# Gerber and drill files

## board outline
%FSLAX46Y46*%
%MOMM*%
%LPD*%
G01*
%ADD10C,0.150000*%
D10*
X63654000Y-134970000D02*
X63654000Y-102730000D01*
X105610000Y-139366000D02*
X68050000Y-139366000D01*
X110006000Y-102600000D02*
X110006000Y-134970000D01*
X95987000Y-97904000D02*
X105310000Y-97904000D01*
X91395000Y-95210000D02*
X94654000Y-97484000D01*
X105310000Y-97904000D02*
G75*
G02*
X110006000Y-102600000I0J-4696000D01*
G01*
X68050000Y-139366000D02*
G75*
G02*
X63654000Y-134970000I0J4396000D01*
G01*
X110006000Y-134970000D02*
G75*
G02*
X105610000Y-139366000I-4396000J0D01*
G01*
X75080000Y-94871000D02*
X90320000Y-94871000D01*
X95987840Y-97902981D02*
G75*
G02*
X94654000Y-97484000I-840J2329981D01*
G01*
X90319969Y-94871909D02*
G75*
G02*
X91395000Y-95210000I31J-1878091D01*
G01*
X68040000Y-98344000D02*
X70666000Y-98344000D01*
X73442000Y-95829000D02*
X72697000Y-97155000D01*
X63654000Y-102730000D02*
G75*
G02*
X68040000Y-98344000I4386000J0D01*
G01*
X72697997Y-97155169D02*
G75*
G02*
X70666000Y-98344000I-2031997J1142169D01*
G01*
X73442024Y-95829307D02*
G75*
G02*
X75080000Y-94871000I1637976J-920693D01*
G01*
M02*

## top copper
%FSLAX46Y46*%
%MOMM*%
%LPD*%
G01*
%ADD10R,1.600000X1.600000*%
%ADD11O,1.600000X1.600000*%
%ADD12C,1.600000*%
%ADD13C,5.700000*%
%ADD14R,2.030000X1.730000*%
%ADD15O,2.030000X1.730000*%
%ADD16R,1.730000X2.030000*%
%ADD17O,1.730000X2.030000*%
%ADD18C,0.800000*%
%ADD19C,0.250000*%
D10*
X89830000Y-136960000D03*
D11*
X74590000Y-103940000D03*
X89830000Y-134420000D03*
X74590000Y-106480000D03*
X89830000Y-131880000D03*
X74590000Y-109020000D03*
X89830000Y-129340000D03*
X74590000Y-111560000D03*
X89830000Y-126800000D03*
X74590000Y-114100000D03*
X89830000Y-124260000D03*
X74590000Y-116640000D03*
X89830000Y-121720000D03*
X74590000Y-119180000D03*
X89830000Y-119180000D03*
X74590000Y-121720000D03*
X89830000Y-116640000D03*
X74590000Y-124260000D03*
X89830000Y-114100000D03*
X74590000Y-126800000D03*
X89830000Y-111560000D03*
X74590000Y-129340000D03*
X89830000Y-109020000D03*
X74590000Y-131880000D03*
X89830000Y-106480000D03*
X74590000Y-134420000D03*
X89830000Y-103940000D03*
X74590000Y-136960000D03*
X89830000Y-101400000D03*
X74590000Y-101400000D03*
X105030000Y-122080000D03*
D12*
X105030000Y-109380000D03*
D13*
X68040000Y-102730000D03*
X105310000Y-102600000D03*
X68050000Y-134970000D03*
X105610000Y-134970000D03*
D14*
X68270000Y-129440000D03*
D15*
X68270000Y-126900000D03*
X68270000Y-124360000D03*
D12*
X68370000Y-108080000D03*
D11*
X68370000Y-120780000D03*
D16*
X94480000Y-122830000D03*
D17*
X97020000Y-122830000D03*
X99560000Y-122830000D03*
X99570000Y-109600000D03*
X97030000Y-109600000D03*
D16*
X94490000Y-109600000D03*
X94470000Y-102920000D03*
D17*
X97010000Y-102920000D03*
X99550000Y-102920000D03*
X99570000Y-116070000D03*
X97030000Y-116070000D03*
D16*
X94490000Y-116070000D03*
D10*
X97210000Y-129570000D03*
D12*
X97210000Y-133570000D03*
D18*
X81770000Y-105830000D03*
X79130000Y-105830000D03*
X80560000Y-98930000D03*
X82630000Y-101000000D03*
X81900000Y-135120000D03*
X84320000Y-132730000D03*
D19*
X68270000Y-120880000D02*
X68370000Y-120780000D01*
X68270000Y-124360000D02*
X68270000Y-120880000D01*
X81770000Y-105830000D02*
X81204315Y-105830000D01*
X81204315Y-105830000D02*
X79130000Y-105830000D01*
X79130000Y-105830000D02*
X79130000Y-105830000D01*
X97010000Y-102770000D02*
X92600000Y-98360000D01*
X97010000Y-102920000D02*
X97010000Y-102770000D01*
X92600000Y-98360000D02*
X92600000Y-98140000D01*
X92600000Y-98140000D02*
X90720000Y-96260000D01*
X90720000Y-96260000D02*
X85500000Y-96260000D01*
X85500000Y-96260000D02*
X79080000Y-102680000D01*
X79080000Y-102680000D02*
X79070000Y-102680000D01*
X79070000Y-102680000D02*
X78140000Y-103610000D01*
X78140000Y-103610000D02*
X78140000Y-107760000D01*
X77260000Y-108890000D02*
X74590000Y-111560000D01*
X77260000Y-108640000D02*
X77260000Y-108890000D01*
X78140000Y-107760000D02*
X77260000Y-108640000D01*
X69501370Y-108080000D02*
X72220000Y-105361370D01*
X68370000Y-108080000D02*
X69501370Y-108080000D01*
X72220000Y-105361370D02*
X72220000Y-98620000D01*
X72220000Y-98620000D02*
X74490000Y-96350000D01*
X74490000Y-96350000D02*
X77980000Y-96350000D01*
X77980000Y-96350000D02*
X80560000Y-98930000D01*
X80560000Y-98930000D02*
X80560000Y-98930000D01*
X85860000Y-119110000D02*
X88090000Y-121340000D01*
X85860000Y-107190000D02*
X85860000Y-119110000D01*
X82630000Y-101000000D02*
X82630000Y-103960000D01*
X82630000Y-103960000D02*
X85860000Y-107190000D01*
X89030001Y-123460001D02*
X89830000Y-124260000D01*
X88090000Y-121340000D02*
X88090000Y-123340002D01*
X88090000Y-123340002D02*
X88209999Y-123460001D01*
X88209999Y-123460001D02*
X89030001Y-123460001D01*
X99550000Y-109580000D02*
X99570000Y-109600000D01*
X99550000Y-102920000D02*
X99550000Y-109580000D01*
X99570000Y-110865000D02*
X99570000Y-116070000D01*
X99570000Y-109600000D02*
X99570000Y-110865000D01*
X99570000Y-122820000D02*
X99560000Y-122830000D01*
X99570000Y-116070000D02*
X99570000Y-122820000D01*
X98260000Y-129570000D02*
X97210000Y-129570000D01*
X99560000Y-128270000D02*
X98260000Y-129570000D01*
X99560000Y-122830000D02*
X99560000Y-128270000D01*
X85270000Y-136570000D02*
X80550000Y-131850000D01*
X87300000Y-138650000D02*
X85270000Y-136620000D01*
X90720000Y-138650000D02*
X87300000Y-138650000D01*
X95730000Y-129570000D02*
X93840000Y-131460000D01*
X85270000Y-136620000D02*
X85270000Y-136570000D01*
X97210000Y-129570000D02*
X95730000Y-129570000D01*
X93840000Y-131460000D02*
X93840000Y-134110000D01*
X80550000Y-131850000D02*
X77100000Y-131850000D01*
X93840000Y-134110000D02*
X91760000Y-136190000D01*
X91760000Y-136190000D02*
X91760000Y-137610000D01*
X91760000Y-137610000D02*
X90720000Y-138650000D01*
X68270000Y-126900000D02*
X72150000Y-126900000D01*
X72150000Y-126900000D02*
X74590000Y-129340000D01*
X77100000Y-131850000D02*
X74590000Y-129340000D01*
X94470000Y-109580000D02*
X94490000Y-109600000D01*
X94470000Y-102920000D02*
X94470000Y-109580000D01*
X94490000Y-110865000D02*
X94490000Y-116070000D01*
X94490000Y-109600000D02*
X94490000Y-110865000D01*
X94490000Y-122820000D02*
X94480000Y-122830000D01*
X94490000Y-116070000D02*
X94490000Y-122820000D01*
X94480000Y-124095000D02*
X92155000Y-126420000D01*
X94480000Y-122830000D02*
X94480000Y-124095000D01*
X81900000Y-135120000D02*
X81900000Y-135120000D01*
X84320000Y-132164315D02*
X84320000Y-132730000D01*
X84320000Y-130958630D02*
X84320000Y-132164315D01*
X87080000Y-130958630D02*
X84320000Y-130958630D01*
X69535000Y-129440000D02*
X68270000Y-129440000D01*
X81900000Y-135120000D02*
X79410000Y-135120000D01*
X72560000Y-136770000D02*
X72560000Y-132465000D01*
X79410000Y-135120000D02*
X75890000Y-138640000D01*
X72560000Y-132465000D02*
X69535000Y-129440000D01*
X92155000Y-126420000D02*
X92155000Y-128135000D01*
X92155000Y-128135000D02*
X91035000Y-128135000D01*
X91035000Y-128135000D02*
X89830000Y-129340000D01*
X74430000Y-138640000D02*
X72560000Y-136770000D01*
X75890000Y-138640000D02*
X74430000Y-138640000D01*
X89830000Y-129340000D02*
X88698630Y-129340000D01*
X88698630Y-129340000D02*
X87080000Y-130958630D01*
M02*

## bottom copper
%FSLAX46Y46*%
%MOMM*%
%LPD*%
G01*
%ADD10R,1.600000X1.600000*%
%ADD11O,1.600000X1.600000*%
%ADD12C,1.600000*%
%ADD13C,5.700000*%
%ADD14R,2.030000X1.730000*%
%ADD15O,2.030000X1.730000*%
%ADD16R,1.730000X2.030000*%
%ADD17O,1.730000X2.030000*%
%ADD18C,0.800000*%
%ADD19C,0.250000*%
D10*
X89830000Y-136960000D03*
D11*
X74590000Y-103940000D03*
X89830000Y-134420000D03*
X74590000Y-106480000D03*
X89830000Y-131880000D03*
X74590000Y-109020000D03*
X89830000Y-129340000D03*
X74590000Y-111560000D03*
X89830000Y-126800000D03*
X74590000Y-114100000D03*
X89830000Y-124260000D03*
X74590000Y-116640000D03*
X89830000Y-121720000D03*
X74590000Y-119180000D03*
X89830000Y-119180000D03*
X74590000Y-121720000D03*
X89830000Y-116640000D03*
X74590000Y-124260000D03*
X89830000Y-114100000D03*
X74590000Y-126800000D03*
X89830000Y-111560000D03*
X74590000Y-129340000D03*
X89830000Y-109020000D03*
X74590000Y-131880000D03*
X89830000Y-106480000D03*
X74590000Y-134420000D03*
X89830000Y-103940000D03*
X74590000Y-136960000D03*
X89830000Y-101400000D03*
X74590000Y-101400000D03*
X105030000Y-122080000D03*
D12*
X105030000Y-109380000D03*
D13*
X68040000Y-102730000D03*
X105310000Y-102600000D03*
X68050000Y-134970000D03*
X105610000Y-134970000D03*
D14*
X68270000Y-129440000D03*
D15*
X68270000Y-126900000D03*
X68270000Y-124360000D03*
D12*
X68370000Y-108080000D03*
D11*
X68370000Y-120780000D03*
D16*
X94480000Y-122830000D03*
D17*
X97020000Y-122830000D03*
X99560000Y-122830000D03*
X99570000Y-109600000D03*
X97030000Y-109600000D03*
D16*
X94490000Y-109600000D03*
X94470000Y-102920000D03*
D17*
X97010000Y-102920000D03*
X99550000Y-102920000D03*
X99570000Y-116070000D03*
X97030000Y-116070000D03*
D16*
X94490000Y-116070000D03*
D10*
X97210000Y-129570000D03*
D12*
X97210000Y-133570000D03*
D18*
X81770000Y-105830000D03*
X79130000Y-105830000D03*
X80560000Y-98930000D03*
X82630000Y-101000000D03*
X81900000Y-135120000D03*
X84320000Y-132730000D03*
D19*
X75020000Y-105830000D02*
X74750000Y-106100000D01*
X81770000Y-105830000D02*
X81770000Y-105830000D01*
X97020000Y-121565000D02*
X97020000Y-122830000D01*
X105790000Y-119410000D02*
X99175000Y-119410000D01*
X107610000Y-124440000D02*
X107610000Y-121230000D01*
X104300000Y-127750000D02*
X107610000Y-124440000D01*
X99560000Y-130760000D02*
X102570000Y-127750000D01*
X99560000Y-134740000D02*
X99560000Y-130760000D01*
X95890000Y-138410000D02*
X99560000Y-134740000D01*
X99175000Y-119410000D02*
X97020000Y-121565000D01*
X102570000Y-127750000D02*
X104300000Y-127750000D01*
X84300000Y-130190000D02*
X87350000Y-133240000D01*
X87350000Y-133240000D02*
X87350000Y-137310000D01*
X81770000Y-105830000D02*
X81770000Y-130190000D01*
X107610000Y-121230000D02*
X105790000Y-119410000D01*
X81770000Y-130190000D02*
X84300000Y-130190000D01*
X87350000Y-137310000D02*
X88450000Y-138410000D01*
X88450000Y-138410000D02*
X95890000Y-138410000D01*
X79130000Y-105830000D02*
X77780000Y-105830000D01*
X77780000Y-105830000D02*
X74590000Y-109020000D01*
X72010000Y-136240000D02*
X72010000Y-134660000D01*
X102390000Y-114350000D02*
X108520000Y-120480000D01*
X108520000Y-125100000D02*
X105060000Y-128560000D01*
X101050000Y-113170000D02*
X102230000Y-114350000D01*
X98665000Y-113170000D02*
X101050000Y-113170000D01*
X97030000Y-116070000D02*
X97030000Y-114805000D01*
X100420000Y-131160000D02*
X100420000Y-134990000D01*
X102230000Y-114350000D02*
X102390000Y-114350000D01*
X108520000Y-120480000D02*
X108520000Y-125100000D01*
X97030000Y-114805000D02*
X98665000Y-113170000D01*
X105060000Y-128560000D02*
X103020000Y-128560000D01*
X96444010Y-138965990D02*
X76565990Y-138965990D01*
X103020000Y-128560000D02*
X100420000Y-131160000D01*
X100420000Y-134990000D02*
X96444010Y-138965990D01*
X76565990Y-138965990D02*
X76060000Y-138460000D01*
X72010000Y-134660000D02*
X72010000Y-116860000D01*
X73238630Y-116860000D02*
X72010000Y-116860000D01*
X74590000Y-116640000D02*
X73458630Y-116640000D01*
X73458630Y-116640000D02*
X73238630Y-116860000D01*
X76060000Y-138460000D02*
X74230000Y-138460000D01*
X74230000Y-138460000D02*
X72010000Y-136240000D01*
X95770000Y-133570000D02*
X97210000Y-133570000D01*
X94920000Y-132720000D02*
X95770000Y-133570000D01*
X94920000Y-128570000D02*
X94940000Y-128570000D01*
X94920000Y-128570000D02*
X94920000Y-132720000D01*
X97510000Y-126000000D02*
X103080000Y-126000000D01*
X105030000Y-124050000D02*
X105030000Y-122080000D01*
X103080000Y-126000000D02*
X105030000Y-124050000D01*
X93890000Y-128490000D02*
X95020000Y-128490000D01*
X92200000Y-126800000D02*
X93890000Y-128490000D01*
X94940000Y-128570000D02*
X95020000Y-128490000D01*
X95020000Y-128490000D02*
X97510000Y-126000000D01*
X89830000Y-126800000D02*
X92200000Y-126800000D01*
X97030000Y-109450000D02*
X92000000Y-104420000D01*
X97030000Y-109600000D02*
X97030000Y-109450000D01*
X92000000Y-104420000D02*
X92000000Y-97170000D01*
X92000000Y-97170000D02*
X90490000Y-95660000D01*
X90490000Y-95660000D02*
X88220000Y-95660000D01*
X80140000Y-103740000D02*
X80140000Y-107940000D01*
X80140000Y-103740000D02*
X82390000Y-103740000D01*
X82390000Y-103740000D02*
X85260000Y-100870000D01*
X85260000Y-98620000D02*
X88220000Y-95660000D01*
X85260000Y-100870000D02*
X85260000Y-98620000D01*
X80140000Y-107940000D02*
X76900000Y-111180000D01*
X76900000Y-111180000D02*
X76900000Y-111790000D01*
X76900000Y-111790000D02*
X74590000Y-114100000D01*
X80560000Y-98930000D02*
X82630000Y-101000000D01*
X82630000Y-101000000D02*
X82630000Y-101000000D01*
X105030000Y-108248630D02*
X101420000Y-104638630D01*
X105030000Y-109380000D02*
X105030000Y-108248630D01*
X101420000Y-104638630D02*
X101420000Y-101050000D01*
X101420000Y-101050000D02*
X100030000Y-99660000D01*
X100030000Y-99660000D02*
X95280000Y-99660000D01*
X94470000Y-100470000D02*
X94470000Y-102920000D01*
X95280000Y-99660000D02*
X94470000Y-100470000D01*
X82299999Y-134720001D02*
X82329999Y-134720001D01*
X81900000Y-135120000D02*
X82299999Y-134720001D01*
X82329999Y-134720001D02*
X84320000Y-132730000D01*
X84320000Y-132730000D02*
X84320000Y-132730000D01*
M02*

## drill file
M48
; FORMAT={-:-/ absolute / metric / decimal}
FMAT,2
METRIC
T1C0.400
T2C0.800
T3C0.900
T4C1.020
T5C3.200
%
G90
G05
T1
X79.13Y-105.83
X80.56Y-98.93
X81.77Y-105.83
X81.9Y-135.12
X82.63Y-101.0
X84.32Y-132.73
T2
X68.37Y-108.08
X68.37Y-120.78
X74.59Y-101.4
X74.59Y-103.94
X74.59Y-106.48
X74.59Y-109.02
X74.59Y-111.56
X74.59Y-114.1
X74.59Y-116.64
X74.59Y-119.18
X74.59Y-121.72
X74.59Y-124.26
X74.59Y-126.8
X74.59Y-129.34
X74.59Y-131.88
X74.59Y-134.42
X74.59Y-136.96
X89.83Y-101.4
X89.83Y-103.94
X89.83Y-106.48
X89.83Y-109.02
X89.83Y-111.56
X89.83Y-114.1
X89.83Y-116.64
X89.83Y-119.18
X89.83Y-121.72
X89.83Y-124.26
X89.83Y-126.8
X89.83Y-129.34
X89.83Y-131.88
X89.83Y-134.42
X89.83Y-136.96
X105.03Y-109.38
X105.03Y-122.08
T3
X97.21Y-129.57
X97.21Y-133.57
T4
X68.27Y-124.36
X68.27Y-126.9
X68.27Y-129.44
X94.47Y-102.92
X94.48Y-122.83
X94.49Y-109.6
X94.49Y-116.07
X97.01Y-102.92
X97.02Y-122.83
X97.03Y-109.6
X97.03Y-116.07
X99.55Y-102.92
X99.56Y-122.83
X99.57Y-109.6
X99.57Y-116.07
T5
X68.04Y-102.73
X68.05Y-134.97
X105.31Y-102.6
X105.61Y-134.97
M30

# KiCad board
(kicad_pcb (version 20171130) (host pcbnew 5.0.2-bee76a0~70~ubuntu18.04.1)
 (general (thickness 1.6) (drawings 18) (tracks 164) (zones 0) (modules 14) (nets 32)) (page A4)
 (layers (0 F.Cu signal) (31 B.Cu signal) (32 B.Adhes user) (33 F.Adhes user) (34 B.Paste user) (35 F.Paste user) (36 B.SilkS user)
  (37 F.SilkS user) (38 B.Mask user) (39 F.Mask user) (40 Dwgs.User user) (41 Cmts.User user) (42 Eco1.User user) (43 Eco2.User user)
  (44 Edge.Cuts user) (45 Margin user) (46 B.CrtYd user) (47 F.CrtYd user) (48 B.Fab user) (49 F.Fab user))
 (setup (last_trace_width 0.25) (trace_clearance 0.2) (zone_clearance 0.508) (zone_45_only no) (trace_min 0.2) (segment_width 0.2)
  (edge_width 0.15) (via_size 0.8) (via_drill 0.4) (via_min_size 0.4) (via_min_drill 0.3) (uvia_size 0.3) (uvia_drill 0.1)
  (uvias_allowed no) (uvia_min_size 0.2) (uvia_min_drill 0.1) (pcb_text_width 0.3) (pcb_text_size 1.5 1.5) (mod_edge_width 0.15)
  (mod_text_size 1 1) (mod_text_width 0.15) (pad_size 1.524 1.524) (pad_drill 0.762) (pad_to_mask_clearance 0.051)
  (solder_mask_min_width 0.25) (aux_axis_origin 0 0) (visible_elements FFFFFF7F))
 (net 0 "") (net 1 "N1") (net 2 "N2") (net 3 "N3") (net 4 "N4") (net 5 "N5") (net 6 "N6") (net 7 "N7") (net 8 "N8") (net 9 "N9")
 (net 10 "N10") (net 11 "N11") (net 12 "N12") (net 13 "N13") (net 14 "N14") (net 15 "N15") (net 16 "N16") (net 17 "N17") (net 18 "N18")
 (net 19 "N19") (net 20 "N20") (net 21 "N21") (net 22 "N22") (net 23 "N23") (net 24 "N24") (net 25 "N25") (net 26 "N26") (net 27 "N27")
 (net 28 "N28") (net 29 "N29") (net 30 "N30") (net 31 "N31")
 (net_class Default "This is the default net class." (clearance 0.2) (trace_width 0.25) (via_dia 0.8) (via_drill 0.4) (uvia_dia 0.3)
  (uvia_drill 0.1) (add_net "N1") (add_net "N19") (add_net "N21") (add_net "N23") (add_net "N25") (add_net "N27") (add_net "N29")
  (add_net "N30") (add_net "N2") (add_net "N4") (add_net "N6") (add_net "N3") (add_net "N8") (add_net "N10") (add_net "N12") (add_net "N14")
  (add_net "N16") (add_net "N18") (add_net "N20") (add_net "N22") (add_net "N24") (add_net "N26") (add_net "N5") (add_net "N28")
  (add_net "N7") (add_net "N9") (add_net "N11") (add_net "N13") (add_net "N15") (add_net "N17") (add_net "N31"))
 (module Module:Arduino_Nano (layer F.Cu) (at 89.83 136.96 180)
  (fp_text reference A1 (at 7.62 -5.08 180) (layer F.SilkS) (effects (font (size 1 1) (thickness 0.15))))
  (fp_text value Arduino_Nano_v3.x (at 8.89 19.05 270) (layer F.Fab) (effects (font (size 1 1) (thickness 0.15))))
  (pad 1 thru_hole rect (at 0 0 180) (size 1.6 1.6) (drill 0.8) (layers *.Cu *.Mask) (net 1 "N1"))
  (pad 17 thru_hole oval (at 15.24 33.02 180) (size 1.6 1.6) (drill 0.8) (layers *.Cu *.Mask) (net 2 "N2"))
  (pad 2 thru_hole oval (at 0 2.54 180) (size 1.6 1.6) (drill 0.8) (layers *.Cu *.Mask) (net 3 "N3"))
  (pad 18 thru_hole oval (at 15.24 30.48 180) (size 1.6 1.6) (drill 0.8) (layers *.Cu *.Mask) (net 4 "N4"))
  (pad 3 thru_hole oval (at 0 5.08 180) (size 1.6 1.6) (drill 0.8) (layers *.Cu *.Mask) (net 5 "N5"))
  (pad 19 thru_hole oval (at 15.24 27.94 180) (size 1.6 1.6) (drill 0.8) (layers *.Cu *.Mask) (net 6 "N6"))
  (pad 4 thru_hole oval (at 0 7.62 180) (size 1.6 1.6) (drill 0.8) (layers *.Cu *.Mask) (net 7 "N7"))
  (pad 20 thru_hole oval (at 15.24 25.4 180) (size 1.6 1.6) (drill 0.8) (layers *.Cu *.Mask) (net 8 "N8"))
  (pad 5 thru_hole oval (at 0 10.16 180) (size 1.6 1.6) (drill 0.8) (layers *.Cu *.Mask) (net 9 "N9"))
  (pad 21 thru_hole oval (at 15.24 22.86 180) (size 1.6 1.6) (drill 0.8) (layers *.Cu *.Mask) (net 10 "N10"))
  (pad 6 thru_hole oval (at 0 12.7 180) (size 1.6 1.6) (drill 0.8) (layers *.Cu *.Mask) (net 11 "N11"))
  (pad 22 thru_hole oval (at 15.24 20.32 180) (size 1.6 1.6) (drill 0.8) (layers *.Cu *.Mask) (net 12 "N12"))
  (pad 7 thru_hole oval (at 0 15.24 180) (size 1.6 1.6) (drill 0.8) (layers *.Cu *.Mask) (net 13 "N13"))
  (pad 23 thru_hole oval (at 15.24 17.78 180) (size 1.6 1.6) (drill 0.8) (layers *.Cu *.Mask) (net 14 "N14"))
  (pad 8 thru_hole oval (at 0 17.78 180) (size 1.6 1.6) (drill 0.8) (layers *.Cu *.Mask) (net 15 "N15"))
  (pad 24 thru_hole oval (at 15.24 15.24 180) (size 1.6 1.6) (drill 0.8) (layers *.Cu *.Mask) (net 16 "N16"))
  (pad 9 thru_hole oval (at 0 20.32 180) (size 1.6 1.6) (drill 0.8) (layers *.Cu *.Mask) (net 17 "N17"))
  (pad 25 thru_hole oval (at 15.24 12.7 180) (size 1.6 1.6) (drill 0.8) (layers *.Cu *.Mask) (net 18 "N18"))
  (pad 10 thru_hole oval (at 0 22.86 180) (size 1.6 1.6) (drill 0.8) (layers *.Cu *.Mask) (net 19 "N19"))
  (pad 26 thru_hole oval (at 15.24 10.16 180) (size 1.6 1.6) (drill 0.8) (layers *.Cu *.Mask) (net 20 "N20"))
  (pad 11 thru_hole oval (at 0 25.4 180) (size 1.6 1.6) (drill 0.8) (layers *.Cu *.Mask) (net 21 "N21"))
  (pad 27 thru_hole oval (at 15.24 7.62 180) (size 1.6 1.6) (drill 0.8) (layers *.Cu *.Mask) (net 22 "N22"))
  (pad 12 thru_hole oval (at 0 27.94 180) (size 1.6 1.6) (drill 0.8) (layers *.Cu *.Mask) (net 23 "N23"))
  (pad 28 thru_hole oval (at 15.24 5.08 180) (size 1.6 1.6) (drill 0.8) (layers *.Cu *.Mask) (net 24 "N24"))
  (pad 13 thru_hole oval (at 0 30.48 180) (size 1.6 1.6) (drill 0.8) (layers *.Cu *.Mask) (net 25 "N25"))
  (pad 29 thru_hole oval (at 15.24 2.54 180) (size 1.6 1.6) (drill 0.8) (layers *.Cu *.Mask) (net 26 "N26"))
  (pad 14 thru_hole oval (at 0 33.02 180) (size 1.6 1.6) (drill 0.8) (layers *.Cu *.Mask) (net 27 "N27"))
  (pad 30 thru_hole oval (at 15.24 0 180) (size 1.6 1.6) (drill 0.8) (layers *.Cu *.Mask) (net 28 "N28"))
  (pad 15 thru_hole oval (at 0 35.56 180) (size 1.6 1.6) (drill 0.8) (layers *.Cu *.Mask) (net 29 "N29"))
  (pad 16 thru_hole oval (at 15.24 35.56 180) (size 1.6 1.6) (drill 0.8) (layers *.Cu *.Mask) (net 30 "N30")))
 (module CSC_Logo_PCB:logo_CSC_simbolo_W (layer F.Cu) (at 81.88 125.63)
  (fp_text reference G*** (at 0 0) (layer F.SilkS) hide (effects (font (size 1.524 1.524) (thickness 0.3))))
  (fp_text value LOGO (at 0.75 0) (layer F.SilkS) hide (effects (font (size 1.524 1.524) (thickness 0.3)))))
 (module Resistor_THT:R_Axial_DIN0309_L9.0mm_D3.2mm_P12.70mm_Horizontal (layer F.Cu) (at 105.03 109.38 270)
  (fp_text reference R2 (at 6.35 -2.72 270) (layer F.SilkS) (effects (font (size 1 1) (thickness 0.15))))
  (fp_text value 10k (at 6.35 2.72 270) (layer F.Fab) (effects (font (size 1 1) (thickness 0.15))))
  (pad 2 thru_hole oval (at 12.7 0 270) (size 1.6 1.6) (drill 0.8) (layers *.Cu *.Mask) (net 9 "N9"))
  (pad 1 thru_hole circle (at 0 0 270) (size 1.6 1.6) (drill 0.8) (layers *.Cu *.Mask) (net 7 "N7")))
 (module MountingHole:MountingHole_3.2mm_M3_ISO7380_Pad (layer F.Cu) (at 68.04 102.73)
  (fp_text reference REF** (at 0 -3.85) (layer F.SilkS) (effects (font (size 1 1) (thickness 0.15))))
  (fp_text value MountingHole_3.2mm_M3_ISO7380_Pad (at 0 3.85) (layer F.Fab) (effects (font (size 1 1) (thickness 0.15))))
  (pad 1 thru_hole circle (at 0 0) (size 5.7 5.7) (drill 3.2) (layers *.Cu *.Mask)))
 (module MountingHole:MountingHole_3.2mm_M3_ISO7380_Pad (layer F.Cu) (at 105.31 102.6)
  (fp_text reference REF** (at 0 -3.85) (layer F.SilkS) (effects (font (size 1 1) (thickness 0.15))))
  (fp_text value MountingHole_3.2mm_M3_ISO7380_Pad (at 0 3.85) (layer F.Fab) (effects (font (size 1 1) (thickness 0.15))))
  (pad 1 thru_hole circle (at 0 0) (size 5.7 5.7) (drill 3.2) (layers *.Cu *.Mask)))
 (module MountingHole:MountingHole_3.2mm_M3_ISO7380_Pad (layer F.Cu) (at 68.05 134.97)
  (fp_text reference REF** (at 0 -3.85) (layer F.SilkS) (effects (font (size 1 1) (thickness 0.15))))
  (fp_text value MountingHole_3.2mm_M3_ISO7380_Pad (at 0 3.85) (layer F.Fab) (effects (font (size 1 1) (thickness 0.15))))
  (pad 1 thru_hole circle (at 0 0) (size 5.7 5.7) (drill 3.2) (layers *.Cu *.Mask)))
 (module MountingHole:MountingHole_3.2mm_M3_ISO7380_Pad (layer F.Cu) (at 105.61 134.97)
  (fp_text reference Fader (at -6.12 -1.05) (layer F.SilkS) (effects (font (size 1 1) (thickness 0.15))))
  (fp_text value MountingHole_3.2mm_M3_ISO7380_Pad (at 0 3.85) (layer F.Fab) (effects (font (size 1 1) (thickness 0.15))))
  (pad 1 thru_hole circle (at 0 0) (size 5.7 5.7) (drill 3.2) (layers *.Cu *.Mask)))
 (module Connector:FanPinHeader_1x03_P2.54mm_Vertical (layer F.Cu) (at 68.27 129.44 90)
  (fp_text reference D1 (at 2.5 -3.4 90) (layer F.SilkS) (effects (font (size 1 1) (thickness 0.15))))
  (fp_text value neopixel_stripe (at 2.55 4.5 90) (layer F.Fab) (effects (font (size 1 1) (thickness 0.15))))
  (pad 1 thru_hole rect (at 0 0 180) (size 2.03 1.73) (drill 1.02) (layers *.Cu *.Mask) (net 7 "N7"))
  (pad 2 thru_hole oval (at 2.54 0 180) (size 2.03 1.73) (drill 1.02) (layers *.Cu *.Mask) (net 22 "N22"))
  (pad 3 thru_hole oval (at 5.08 0 180) (size 2.03 1.73) (drill 1.02) (layers *.Cu *.Mask) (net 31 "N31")))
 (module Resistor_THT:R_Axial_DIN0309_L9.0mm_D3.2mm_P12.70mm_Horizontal (layer F.Cu) (at 68.37 108.08 270)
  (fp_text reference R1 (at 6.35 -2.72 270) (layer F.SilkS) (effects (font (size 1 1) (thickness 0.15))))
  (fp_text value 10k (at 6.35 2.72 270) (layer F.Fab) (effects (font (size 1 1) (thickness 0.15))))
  (pad 1 thru_hole circle (at 0 0 270) (size 1.6 1.6) (drill 0.8) (layers *.Cu *.Mask) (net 11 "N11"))
  (pad 2 thru_hole oval (at 12.7 0 270) (size 1.6 1.6) (drill 0.8) (layers *.Cu *.Mask) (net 31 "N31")))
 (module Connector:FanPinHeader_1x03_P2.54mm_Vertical (layer F.Cu) (at 94.48 122.83)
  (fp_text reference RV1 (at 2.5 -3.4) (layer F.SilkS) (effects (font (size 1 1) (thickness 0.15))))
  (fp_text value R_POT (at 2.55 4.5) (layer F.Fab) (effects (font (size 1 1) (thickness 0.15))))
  (pad 1 thru_hole rect (at 0 0 90) (size 2.03 1.73) (drill 1.02) (layers *.Cu *.Mask) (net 7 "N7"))
  (pad 2 thru_hole oval (at 2.54 0 90) (size 2.03 1.73) (drill 1.02) (layers *.Cu *.Mask) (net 6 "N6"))
  (pad 3 thru_hole oval (at 5.08 0 90) (size 2.03 1.73) (drill 1.02) (layers *.Cu *.Mask) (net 22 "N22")))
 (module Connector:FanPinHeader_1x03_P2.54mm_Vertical (layer F.Cu) (at 94.49 109.6)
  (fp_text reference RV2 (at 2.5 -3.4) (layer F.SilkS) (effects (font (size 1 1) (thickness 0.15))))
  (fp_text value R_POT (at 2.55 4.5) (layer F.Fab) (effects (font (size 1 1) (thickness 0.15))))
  (pad 3 thru_hole oval (at 5.08 0 90) (size 2.03 1.73) (drill 1.02) (layers *.Cu *.Mask) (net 22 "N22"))
  (pad 2 thru_hole oval (at 2.54 0 90) (size 2.03 1.73) (drill 1.02) (layers *.Cu *.Mask) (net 10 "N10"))
  (pad 1 thru_hole rect (at 0 0 90) (size 2.03 1.73) (drill 1.02) (layers *.Cu *.Mask) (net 7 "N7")))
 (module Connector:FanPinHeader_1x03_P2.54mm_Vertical (layer F.Cu) (at 94.47 102.92)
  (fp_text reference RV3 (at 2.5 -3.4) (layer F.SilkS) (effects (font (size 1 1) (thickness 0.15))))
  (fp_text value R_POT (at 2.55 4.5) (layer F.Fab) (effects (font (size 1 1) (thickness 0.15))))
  (pad 1 thru_hole rect (at 0 0 90) (size 2.03 1.73) (drill 1.02) (layers *.Cu *.Mask) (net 7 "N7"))
  (pad 2 thru_hole oval (at 2.54 0 90) (size 2.03 1.73) (drill 1.02) (layers *.Cu *.Mask) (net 8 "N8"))
  (pad 3 thru_hole oval (at 5.08 0 90) (size 2.03 1.73) (drill 1.02) (layers *.Cu *.Mask) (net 22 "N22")))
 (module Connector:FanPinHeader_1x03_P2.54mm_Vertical (layer F.Cu) (at 94.49 116.07)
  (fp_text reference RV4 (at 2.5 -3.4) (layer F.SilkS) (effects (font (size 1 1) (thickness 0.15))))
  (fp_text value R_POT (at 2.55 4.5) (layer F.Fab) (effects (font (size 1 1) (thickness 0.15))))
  (pad 3 thru_hole oval (at 5.08 0 90) (size 2.03 1.73) (drill 1.02) (layers *.Cu *.Mask) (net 22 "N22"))
  (pad 2 thru_hole oval (at 2.54 0 90) (size 2.03 1.73) (drill 1.02) (layers *.Cu *.Mask) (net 12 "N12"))
  (pad 1 thru_hole rect (at 0 0 90) (size 2.03 1.73) (drill 1.02) (layers *.Cu *.Mask) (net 7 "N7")))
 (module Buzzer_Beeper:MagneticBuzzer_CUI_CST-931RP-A (layer F.Cu) (at 97.21 129.57)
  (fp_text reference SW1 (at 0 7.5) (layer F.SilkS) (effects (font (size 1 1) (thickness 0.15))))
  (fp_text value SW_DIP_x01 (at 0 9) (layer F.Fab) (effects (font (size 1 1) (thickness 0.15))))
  (pad 1 thru_hole rect (at 0 0) (size 1.6 1.6) (drill 0.9) (layers *.Cu *.Mask) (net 22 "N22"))
  (pad 2 thru_hole circle (at 0 4) (size 1.6 1.6) (drill 0.9) (layers *.Cu *.Mask) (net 9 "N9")))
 (gr_line (start 63.654 134.97) (end 63.654 102.73) (angle 90) (layer Edge.Cuts) (width 0.15))
 (gr_line (start 105.61 139.366) (end 68.05 139.366) (angle 90) (layer Edge.Cuts) (width 0.15))
 (gr_line (start 110.006 102.6) (end 110.006 134.97) (angle 90) (layer Edge.Cuts) (width 0.15))
 (gr_line (start 95.987 97.904) (end 105.31 97.904) (angle 90) (layer Edge.Cuts) (width 0.15))
 (gr_line (start 91.395 95.21) (end 94.654 97.484) (angle 90) (layer Edge.Cuts) (width 0.15))
 (gr_arc (start 105.31 102.6) (end 110.006 102.6) (angle -90) (layer Edge.Cuts) (width 0.15))
 (gr_arc (start 68.05 134.97) (end 63.654 134.97) (angle -90) (layer Edge.Cuts) (width 0.15))
 (gr_arc (start 105.61 134.97) (end 105.61 139.366) (angle -90) (layer Edge.Cuts) (width 0.15))
 (gr_line (start 75.08 94.871) (end 90.32 94.871) (angle 90) (layer Edge.Cuts) (width 0.15))
 (gr_arc (start 95.987 95.573) (end 94.654 97.484) (angle -34.918) (layer Edge.Cuts) (width 0.15))
 (gr_arc (start 90.32 96.75) (end 91.395 95.21) (angle -34.918) (layer Edge.Cuts) (width 0.15))
 (gr_line (start 68.04 98.344) (end 70.666 98.344) (angle 90) (layer Edge.Cuts) (width 0.15))
 (gr_line (start 73.442 95.829) (end 72.697 97.155) (angle 90) (layer Edge.Cuts) (width 0.15))
 (gr_arc (start 68.04 102.73) (end 68.04 98.344) (angle -90) (layer Edge.Cuts) (width 0.15))
 (gr_arc (start 70.666 96.013) (end 70.666 98.344) (angle -60.66) (layer Edge.Cuts) (width 0.15))
 (gr_arc (start 75.08 96.75) (end 75.08 94.871) (angle -60.66) (layer Edge.Cuts) (width 0.15))
 (segment (start 68.27 120.88) (end 68.37 120.78) (width 0.25) (layer F.Cu) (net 31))
 (segment (start 68.27 124.36) (end 68.27 120.88) (width 0.25) (layer F.Cu) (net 31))
 (segment (start 75.02 105.83) (end 74.75 106.1) (width 0.25) (layer B.Cu) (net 4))
 (segment (start 81.77 105.83) (end 81.77 105.83) (width 0.25) (layer B.Cu) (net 6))
 (via (at 81.77 105.83) (size 0.8) (drill 0.4) (layers F.Cu B.Cu) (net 6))
 (segment (start 81.77 105.83) (end 81.204315 105.83) (width 0.25) (layer F.Cu) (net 6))
 (segment (start 81.204315 105.83) (end 79.13 105.83) (width 0.25) (layer F.Cu) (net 6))
 (segment (start 79.13 105.83) (end 79.13 105.83) (width 0.25) (layer F.Cu) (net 6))
 (via (at 79.13 105.83) (size 0.8) (drill 0.4) (layers F.Cu B.Cu) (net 6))
 (segment (start 97.02 121.565) (end 97.02 122.83) (width 0.25) (layer B.Cu) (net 6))
 (segment (start 105.79 119.41) (end 99.175 119.41) (width 0.25) (layer B.Cu) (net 6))
 (segment (start 107.61 124.44) (end 107.61 121.23) (width 0.25) (layer B.Cu) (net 6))
 (segment (start 104.3 127.75) (end 107.61 124.44) (width 0.25) (layer B.Cu) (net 6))
 (segment (start 99.56 130.76) (end 102.57 127.75) (width 0.25) (layer B.Cu) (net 6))
 (segment (start 99.56 134.74) (end 99.56 130.76) (width 0.25) (layer B.Cu) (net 6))
 (segment (start 95.89 138.41) (end 99.56 134.74) (width 0.25) (layer B.Cu) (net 6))
 (segment (start 99.175 119.41) (end 97.02 121.565) (width 0.25) (layer B.Cu) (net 6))
 (segment (start 102.57 127.75) (end 104.3 127.75) (width 0.25) (layer B.Cu) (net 6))
 (segment (start 84.3 130.19) (end 87.35 133.24) (width 0.25) (layer B.Cu) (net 6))
 (segment (start 87.35 133.24) (end 87.35 137.31) (width 0.25) (layer B.Cu) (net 6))
 (segment (start 81.77 105.83) (end 81.77 130.19) (width 0.25) (layer B.Cu) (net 6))
 (segment (start 107.61 121.23) (end 105.79 119.41) (width 0.25) (layer B.Cu) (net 6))
 (segment (start 81.77 130.19) (end 84.3 130.19) (width 0.25) (layer B.Cu) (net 6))
 (segment (start 87.35 137.31) (end 88.45 138.41) (width 0.25) (layer B.Cu) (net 6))
 (segment (start 88.45 138.41) (end 95.89 138.41) (width 0.25) (layer B.Cu) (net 6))
 (segment (start 79.13 105.83) (end 77.78 105.83) (width 0.25) (layer B.Cu) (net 6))
 (segment (start 77.78 105.83) (end 74.59 109.02) (width 0.25) (layer B.Cu) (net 6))
 (segment (start 72.01 136.24) (end 72.01 134.66) (width 0.25) (layer B.Cu) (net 12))
 (segment (start 102.39 114.35) (end 108.52 120.48) (width 0.25) (layer B.Cu) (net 12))
 (segment (start 108.52 125.1) (end 105.06 128.56) (width 0.25) (layer B.Cu) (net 12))
 (segment (start 101.05 113.17) (end 102.23 114.35) (width 0.25) (layer B.Cu) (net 12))
 (segment (start 98.665 113.17) (end 101.05 113.17) (width 0.25) (layer B.Cu) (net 12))
 (segment (start 97.03 116.07) (end 97.03 114.805) (width 0.25) (layer B.Cu) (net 12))
 (segment (start 100.42 131.16) (end 100.42 134.99) (width 0.25) (layer B.Cu) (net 12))
 (segment (start 102.23 114.35) (end 102.39 114.35) (width 0.25) (layer B.Cu) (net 12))
 (segment (start 108.52 120.48) (end 108.52 125.1) (width 0.25) (layer B.Cu) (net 12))
 (segment (start 97.03 114.805) (end 98.665 113.17) (width 0.25) (layer B.Cu) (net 12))
 (segment (start 105.06 128.56) (end 103.02 128.56) (width 0.25) (layer B.Cu) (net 12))
 (segment (start 96.44401 138.96599) (end 76.56599 138.96599) (width 0.25) (layer B.Cu) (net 12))
 (segment (start 103.02 128.56) (end 100.42 131.16) (width 0.25) (layer B.Cu) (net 12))
 (segment (start 100.42 134.99) (end 96.44401 138.96599) (width 0.25) (layer B.Cu) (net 12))
 (segment (start 76.56599 138.96599) (end 76.06 138.46) (width 0.25) (layer B.Cu) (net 12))
 (segment (start 72.01 134.66) (end 72.01 116.86) (width 0.25) (layer B.Cu) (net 12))
 (segment (start 73.23863 116.86) (end 72.01 116.86) (width 0.25) (layer B.Cu) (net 12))
 (segment (start 74.59 116.64) (end 73.45863 116.64) (width 0.25) (layer B.Cu) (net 12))
 (segment (start 73.45863 116.64) (end 73.23863 116.86) (width 0.25) (layer B.Cu) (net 12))
 (segment (start 76.06 138.46) (end 74.23 138.46) (width 0.25) (layer B.Cu) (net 12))
 (segment (start 74.23 138.46) (end 72.01 136.24) (width 0.25) (layer B.Cu) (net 12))
 (segment (start 97.01 102.77) (end 92.6 98.36) (width 0.25) (layer F.Cu) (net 8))
 (segment (start 97.01 102.92) (end 97.01 102.77) (width 0.25) (layer F.Cu) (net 8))
 (segment (start 92.6 98.36) (end 92.6 98.14) (width 0.25) (layer F.Cu) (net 8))
 (segment (start 92.6 98.14) (end 90.72 96.26) (width 0.25) (layer F.Cu) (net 8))
 (segment (start 90.72 96.26) (end 85.5 96.26) (width 0.25) (layer F.Cu) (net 8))
 (segment (start 85.5 96.26) (end 79.08 102.68) (width 0.25) (layer F.Cu) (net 8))
 (segment (start 79.08 102.68) (end 79.07 102.68) (width 0.25) (layer F.Cu) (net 8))
 (segment (start 79.07 102.68) (end 78.14 103.61) (width 0.25) (layer F.Cu) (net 8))
 (segment (start 78.14 103.61) (end 78.14 107.76) (width 0.25) (layer F.Cu) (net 8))
 (segment (start 77.26 108.89) (end 74.59 111.56) (width 0.25) (layer F.Cu) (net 8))
 (segment (start 77.26 108.64) (end 77.26 108.89) (width 0.25) (layer F.Cu) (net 8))
 (segment (start 78.14 107.76) (end 77.26 108.64) (width 0.25) (layer F.Cu) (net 8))
 (segment (start 95.77 133.57) (end 97.21 133.57) (width 0.25) (layer B.Cu) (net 9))
 (segment (start 94.92 132.72) (end 95.77 133.57) (width 0.25) (layer B.Cu) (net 9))
 (segment (start 94.92 128.57) (end 94.94 128.57) (width 0.25) (layer B.Cu) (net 9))
 (segment (start 94.92 128.57) (end 94.92 132.72) (width 0.25) (layer B.Cu) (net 9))
 (segment (start 97.51 126) (end 103.08 126) (width 0.25) (layer B.Cu) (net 9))
 (segment (start 105.03 124.05) (end 105.03 122.08) (width 0.25) (layer B.Cu) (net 9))
 (segment (start 103.08 126) (end 105.03 124.05) (width 0.25) (layer B.Cu) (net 9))
 (segment (start 93.89 128.49) (end 95.02 128.49) (width 0.25) (layer B.Cu) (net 9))
 (segment (start 92.2 126.8) (end 93.89 128.49) (width 0.25) (layer B.Cu) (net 9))
 (segment (start 94.94 128.57) (end 95.02 128.49) (width 0.25) (layer B.Cu) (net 9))
 (segment (start 95.02 128.49) (end 97.51 126) (width 0.25) (layer B.Cu) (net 9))
 (segment (start 89.83 126.8) (end 92.2 126.8) (width 0.25) (layer B.Cu) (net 9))
 (segment (start 97.03 109.45) (end 92 104.42) (width 0.25) (layer B.Cu) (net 10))
 (segment (start 97.03 109.6) (end 97.03 109.45) (width 0.25) (layer B.Cu) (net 10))
 (segment (start 92 104.42) (end 92 97.17) (width 0.25) (layer B.Cu) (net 10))
 (segment (start 92 97.17) (end 90.49 95.66) (width 0.25) (layer B.Cu) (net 10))
 (segment (start 90.49 95.66) (end 88.22 95.66) (width 0.25) (layer B.Cu) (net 10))
 (segment (start 80.14 103.74) (end 80.14 107.94) (width 0.25) (layer B.Cu) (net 10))
 (segment (start 80.14 103.74) (end 82.39 103.74) (width 0.25) (layer B.Cu) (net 10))
 (segment (start 82.39 103.74) (end 85.26 100.87) (width 0.25) (layer B.Cu) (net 10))
 (segment (start 85.26 98.62) (end 88.22 95.66) (width 0.25) (layer B.Cu) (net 10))
 (segment (start 85.26 100.87) (end 85.26 98.62) (width 0.25) (layer B.Cu) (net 10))
 (segment (start 80.14 107.94) (end 76.9 111.18) (width 0.25) (layer B.Cu) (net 10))
 (segment (start 76.9 111.18) (end 76.9 111.79) (width 0.25) (layer B.Cu) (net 10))
 (segment (start 76.9 111.79) (end 74.59 114.1) (width 0.25) (layer B.Cu) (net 10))
 (segment (start 69.50137 108.08) (end 72.22 105.36137) (width 0.25) (layer F.Cu) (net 11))
 (segment (start 68.37 108.08) (end 69.50137 108.08) (width 0.25) (layer F.Cu) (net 11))
 (segment (start 72.22 105.36137) (end 72.22 98.62) (width 0.25) (layer F.Cu) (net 11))
 (segment (start 72.22 98.62) (end 74.49 96.35) (width 0.25) (layer F.Cu) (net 11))
 (segment (start 74.49 96.35) (end 77.98 96.35) (width 0.25) (layer F.Cu) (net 11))
 (segment (start 77.98 96.35) (end 80.56 98.93) (width 0.25) (layer F.Cu) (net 11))
 (segment (start 80.56 98.93) (end 80.56 98.93) (width 0.25) (layer F.Cu) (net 11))
 (via (at 80.56 98.93) (size 0.8) (drill 0.4) (layers F.Cu B.Cu) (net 11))
 (segment (start 80.56 98.93) (end 82.63 101) (width 0.25) (layer B.Cu) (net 11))
 (segment (start 82.63 101) (end 82.63 101) (width 0.25) (layer B.Cu) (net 11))
 (via (at 82.63 101) (size 0.8) (drill 0.4) (layers F.Cu B.Cu) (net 11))
 (segment (start 85.86 119.11) (end 88.09 121.34) (width 0.25) (layer F.Cu) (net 11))
 (segment (start 85.86 107.19) (end 85.86 119.11) (width 0.25) (layer F.Cu) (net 11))
 (segment (start 82.63 101) (end 82.63 103.96) (width 0.25) (layer F.Cu) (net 11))
 (segment (start 82.63 103.96) (end 85.86 107.19) (width 0.25) (layer F.Cu) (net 11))
 (segment (start 89.030001 123.460001) (end 89.83 124.26) (width 0.25) (layer F.Cu) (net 11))
 (segment (start 88.09 121.34) (end 88.09 123.340002) (width 0.25) (layer F.Cu) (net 11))
 (segment (start 88.09 123.340002) (end 88.209999 123.460001) (width 0.25) (layer F.Cu) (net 11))
 (segment (start 88.209999 123.460001) (end 89.030001 123.460001) (width 0.25) (layer F.Cu) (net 11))
 (segment (start 99.55 109.58) (end 99.57 109.6) (width 0.25) (layer F.Cu) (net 22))
 (segment (start 99.55 102.92) (end 99.55 109.58) (width 0.25) (layer F.Cu) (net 22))
 (segment (start 99.57 110.865) (end 99.57 116.07) (width 0.25) (layer F.Cu) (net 22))
 (segment (start 99.57 109.6) (end 99.57 110.865) (width 0.25) (layer F.Cu) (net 22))
 (segment (start 99.57 122.82) (end 99.56 122.83) (width 0.25) (layer F.Cu) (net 22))
 (segment (start 99.57 116.07) (end 99.57 122.82) (width 0.25) (layer F.Cu) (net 22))
 (segment (start 98.26 129.57) (end 97.21 129.57) (width 0.25) (layer F.Cu) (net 22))
 (segment (start 99.56 128.27) (end 98.26 129.57) (width 0.25) (layer F.Cu) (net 22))
 (segment (start 99.56 122.83) (end 99.56 128.27) (width 0.25) (layer F.Cu) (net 22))
 (segment (start 85.27 136.57) (end 80.55 131.85) (width 0.25) (layer F.Cu) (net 22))
 (segment (start 87.3 138.65) (end 85.27 136.62) (width 0.25) (layer F.Cu) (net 22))
 (segment (start 90.72 138.65) (end 87.3 138.65) (width 0.25) (layer F.Cu) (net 22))
 (segment (start 95.73 129.57) (end 93.84 131.46) (width 0.25) (layer F.Cu) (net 22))
 (segment (start 85.27 136.62) (end 85.27 136.57) (width 0.25) (layer F.Cu) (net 22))
 (segment (start 97.21 129.57) (end 95.73 129.57) (width 0.25) (layer F.Cu) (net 22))
 (segment (start 93.84 131.46) (end 93.84 134.11) (width 0.25) (layer F.Cu) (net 22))
 (segment (start 80.55 131.85) (end 77.1 131.85) (width 0.25) (layer F.Cu) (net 22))
 (segment (start 93.84 134.11) (end 91.76 136.19) (width 0.25) (layer F.Cu) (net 22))
 (segment (start 91.76 136.19) (end 91.76 137.61) (width 0.25) (layer F.Cu) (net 22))
 (segment (start 91.76 137.61) (end 90.72 138.65) (width 0.25) (layer F.Cu) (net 22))
 (segment (start 68.27 126.9) (end 72.15 126.9) (width 0.25) (layer F.Cu) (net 22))
 (segment (start 72.15 126.9) (end 74.59 129.34) (width 0.25) (layer F.Cu) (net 22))
 (segment (start 77.1 131.85) (end 74.59 129.34) (width 0.25) (layer F.Cu) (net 22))
 (segment (start 94.47 109.58) (end 94.49 109.6) (width 0.25) (layer F.Cu) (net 7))
 (segment (start 94.47 102.92) (end 94.47 109.58) (width 0.25) (layer F.Cu) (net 7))
 (segment (start 94.49 110.865) (end 94.49 116.07) (width 0.25) (layer F.Cu) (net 7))
 (segment (start 94.49 109.6) (end 94.49 110.865) (width 0.25) (layer F.Cu) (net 7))
 (segment (start 94.49 122.82) (end 94.48 122.83) (width 0.25) (layer F.Cu) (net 7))
 (segment (start 94.49 116.07) (end 94.49 122.82) (width 0.25) (layer F.Cu) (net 7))
 (segment (start 94.48 124.095) (end 92.155 126.42) (width 0.25) (layer F.Cu) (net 7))
 (segment (start 94.48 122.83) (end 94.48 124.095) (width 0.25) (layer F.Cu) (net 7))
 (segment (start 105.03 108.24863) (end 101.42 104.63863) (width 0.25) (layer B.Cu) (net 7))
 (segment (start 105.03 109.38) (end 105.03 108.24863) (width 0.25) (layer B.Cu) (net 7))
 (segment (start 101.42 104.63863) (end 101.42 101.05) (width 0.25) (layer B.Cu) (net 7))
 (segment (start 101.42 101.05) (end 100.03 99.66) (width 0.25) (layer B.Cu) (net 7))
 (segment (start 100.03 99.66) (end 95.28 99.66) (width 0.25) (layer B.Cu) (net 7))
 (segment (start 94.47 100.47) (end 94.47 102.92) (width 0.25) (layer B.Cu) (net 7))
 (segment (start 95.28 99.66) (end 94.47 100.47) (width 0.25) (layer B.Cu) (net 7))
 (segment (start 81.9 135.12) (end 81.9 135.12) (width 0.25) (layer F.Cu) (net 7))
 (via (at 81.9 135.12) (size 0.8) (drill 0.4) (layers F.Cu B.Cu) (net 7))
 (segment (start 82.299999 134.720001) (end 82.329999 134.720001) (width 0.25) (layer B.Cu) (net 7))
 (segment (start 81.9 135.12) (end 82.299999 134.720001) (width 0.25) (layer B.Cu) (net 7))
 (segment (start 82.329999 134.720001) (end 84.32 132.73) (width 0.25) (layer B.Cu) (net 7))
 (segment (start 84.32 132.73) (end 84.32 132.73) (width 0.25) (layer B.Cu) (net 7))
 (via (at 84.32 132.73) (size 0.8) (drill 0.4) (layers F.Cu B.Cu) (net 7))
 (segment (start 84.32 132.164315) (end 84.32 132.73) (width 0.25) (layer F.Cu) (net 7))
 (segment (start 84.32 130.95863) (end 84.32 132.164315) (width 0.25) (layer F.Cu) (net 7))
 (segment (start 87.08 130.95863) (end 84.32 130.95863) (width 0.25) (layer F.Cu) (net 7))
 (segment (start 69.535 129.44) (end 68.27 129.44) (width 0.25) (layer F.Cu) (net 7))
 (segment (start 81.9 135.12) (end 79.41 135.12) (width 0.25) (layer F.Cu) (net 7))
 (segment (start 72.56 136.77) (end 72.56 132.465) (width 0.25) (layer F.Cu) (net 7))
 (segment (start 79.41 135.12) (end 75.89 138.64) (width 0.25) (layer F.Cu) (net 7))
 (segment (start 72.56 132.465) (end 69.535 129.44) (width 0.25) (layer F.Cu) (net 7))
 (segment (start 92.155 126.42) (end 92.155 128.135) (width 0.25) (layer F.Cu) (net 7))
 (segment (start 92.155 128.135) (end 91.035 128.135) (width 0.25) (layer F.Cu) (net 7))
 (segment (start 91.035 128.135) (end 89.83 129.34) (width 0.25) (layer F.Cu) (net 7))
 (segment (start 74.43 138.64) (end 72.56 136.77) (width 0.25) (layer F.Cu) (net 7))
 (segment (start 75.89 138.64) (end 74.43 138.64) (width 0.25) (layer F.Cu) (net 7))
 (segment (start 89.83 129.34) (end 88.69863 129.34) (width 0.25) (layer F.Cu) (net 7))
 (segment (start 88.69863 129.34) (end 87.08 130.95863) (width 0.25) (layer F.Cu) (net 7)))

